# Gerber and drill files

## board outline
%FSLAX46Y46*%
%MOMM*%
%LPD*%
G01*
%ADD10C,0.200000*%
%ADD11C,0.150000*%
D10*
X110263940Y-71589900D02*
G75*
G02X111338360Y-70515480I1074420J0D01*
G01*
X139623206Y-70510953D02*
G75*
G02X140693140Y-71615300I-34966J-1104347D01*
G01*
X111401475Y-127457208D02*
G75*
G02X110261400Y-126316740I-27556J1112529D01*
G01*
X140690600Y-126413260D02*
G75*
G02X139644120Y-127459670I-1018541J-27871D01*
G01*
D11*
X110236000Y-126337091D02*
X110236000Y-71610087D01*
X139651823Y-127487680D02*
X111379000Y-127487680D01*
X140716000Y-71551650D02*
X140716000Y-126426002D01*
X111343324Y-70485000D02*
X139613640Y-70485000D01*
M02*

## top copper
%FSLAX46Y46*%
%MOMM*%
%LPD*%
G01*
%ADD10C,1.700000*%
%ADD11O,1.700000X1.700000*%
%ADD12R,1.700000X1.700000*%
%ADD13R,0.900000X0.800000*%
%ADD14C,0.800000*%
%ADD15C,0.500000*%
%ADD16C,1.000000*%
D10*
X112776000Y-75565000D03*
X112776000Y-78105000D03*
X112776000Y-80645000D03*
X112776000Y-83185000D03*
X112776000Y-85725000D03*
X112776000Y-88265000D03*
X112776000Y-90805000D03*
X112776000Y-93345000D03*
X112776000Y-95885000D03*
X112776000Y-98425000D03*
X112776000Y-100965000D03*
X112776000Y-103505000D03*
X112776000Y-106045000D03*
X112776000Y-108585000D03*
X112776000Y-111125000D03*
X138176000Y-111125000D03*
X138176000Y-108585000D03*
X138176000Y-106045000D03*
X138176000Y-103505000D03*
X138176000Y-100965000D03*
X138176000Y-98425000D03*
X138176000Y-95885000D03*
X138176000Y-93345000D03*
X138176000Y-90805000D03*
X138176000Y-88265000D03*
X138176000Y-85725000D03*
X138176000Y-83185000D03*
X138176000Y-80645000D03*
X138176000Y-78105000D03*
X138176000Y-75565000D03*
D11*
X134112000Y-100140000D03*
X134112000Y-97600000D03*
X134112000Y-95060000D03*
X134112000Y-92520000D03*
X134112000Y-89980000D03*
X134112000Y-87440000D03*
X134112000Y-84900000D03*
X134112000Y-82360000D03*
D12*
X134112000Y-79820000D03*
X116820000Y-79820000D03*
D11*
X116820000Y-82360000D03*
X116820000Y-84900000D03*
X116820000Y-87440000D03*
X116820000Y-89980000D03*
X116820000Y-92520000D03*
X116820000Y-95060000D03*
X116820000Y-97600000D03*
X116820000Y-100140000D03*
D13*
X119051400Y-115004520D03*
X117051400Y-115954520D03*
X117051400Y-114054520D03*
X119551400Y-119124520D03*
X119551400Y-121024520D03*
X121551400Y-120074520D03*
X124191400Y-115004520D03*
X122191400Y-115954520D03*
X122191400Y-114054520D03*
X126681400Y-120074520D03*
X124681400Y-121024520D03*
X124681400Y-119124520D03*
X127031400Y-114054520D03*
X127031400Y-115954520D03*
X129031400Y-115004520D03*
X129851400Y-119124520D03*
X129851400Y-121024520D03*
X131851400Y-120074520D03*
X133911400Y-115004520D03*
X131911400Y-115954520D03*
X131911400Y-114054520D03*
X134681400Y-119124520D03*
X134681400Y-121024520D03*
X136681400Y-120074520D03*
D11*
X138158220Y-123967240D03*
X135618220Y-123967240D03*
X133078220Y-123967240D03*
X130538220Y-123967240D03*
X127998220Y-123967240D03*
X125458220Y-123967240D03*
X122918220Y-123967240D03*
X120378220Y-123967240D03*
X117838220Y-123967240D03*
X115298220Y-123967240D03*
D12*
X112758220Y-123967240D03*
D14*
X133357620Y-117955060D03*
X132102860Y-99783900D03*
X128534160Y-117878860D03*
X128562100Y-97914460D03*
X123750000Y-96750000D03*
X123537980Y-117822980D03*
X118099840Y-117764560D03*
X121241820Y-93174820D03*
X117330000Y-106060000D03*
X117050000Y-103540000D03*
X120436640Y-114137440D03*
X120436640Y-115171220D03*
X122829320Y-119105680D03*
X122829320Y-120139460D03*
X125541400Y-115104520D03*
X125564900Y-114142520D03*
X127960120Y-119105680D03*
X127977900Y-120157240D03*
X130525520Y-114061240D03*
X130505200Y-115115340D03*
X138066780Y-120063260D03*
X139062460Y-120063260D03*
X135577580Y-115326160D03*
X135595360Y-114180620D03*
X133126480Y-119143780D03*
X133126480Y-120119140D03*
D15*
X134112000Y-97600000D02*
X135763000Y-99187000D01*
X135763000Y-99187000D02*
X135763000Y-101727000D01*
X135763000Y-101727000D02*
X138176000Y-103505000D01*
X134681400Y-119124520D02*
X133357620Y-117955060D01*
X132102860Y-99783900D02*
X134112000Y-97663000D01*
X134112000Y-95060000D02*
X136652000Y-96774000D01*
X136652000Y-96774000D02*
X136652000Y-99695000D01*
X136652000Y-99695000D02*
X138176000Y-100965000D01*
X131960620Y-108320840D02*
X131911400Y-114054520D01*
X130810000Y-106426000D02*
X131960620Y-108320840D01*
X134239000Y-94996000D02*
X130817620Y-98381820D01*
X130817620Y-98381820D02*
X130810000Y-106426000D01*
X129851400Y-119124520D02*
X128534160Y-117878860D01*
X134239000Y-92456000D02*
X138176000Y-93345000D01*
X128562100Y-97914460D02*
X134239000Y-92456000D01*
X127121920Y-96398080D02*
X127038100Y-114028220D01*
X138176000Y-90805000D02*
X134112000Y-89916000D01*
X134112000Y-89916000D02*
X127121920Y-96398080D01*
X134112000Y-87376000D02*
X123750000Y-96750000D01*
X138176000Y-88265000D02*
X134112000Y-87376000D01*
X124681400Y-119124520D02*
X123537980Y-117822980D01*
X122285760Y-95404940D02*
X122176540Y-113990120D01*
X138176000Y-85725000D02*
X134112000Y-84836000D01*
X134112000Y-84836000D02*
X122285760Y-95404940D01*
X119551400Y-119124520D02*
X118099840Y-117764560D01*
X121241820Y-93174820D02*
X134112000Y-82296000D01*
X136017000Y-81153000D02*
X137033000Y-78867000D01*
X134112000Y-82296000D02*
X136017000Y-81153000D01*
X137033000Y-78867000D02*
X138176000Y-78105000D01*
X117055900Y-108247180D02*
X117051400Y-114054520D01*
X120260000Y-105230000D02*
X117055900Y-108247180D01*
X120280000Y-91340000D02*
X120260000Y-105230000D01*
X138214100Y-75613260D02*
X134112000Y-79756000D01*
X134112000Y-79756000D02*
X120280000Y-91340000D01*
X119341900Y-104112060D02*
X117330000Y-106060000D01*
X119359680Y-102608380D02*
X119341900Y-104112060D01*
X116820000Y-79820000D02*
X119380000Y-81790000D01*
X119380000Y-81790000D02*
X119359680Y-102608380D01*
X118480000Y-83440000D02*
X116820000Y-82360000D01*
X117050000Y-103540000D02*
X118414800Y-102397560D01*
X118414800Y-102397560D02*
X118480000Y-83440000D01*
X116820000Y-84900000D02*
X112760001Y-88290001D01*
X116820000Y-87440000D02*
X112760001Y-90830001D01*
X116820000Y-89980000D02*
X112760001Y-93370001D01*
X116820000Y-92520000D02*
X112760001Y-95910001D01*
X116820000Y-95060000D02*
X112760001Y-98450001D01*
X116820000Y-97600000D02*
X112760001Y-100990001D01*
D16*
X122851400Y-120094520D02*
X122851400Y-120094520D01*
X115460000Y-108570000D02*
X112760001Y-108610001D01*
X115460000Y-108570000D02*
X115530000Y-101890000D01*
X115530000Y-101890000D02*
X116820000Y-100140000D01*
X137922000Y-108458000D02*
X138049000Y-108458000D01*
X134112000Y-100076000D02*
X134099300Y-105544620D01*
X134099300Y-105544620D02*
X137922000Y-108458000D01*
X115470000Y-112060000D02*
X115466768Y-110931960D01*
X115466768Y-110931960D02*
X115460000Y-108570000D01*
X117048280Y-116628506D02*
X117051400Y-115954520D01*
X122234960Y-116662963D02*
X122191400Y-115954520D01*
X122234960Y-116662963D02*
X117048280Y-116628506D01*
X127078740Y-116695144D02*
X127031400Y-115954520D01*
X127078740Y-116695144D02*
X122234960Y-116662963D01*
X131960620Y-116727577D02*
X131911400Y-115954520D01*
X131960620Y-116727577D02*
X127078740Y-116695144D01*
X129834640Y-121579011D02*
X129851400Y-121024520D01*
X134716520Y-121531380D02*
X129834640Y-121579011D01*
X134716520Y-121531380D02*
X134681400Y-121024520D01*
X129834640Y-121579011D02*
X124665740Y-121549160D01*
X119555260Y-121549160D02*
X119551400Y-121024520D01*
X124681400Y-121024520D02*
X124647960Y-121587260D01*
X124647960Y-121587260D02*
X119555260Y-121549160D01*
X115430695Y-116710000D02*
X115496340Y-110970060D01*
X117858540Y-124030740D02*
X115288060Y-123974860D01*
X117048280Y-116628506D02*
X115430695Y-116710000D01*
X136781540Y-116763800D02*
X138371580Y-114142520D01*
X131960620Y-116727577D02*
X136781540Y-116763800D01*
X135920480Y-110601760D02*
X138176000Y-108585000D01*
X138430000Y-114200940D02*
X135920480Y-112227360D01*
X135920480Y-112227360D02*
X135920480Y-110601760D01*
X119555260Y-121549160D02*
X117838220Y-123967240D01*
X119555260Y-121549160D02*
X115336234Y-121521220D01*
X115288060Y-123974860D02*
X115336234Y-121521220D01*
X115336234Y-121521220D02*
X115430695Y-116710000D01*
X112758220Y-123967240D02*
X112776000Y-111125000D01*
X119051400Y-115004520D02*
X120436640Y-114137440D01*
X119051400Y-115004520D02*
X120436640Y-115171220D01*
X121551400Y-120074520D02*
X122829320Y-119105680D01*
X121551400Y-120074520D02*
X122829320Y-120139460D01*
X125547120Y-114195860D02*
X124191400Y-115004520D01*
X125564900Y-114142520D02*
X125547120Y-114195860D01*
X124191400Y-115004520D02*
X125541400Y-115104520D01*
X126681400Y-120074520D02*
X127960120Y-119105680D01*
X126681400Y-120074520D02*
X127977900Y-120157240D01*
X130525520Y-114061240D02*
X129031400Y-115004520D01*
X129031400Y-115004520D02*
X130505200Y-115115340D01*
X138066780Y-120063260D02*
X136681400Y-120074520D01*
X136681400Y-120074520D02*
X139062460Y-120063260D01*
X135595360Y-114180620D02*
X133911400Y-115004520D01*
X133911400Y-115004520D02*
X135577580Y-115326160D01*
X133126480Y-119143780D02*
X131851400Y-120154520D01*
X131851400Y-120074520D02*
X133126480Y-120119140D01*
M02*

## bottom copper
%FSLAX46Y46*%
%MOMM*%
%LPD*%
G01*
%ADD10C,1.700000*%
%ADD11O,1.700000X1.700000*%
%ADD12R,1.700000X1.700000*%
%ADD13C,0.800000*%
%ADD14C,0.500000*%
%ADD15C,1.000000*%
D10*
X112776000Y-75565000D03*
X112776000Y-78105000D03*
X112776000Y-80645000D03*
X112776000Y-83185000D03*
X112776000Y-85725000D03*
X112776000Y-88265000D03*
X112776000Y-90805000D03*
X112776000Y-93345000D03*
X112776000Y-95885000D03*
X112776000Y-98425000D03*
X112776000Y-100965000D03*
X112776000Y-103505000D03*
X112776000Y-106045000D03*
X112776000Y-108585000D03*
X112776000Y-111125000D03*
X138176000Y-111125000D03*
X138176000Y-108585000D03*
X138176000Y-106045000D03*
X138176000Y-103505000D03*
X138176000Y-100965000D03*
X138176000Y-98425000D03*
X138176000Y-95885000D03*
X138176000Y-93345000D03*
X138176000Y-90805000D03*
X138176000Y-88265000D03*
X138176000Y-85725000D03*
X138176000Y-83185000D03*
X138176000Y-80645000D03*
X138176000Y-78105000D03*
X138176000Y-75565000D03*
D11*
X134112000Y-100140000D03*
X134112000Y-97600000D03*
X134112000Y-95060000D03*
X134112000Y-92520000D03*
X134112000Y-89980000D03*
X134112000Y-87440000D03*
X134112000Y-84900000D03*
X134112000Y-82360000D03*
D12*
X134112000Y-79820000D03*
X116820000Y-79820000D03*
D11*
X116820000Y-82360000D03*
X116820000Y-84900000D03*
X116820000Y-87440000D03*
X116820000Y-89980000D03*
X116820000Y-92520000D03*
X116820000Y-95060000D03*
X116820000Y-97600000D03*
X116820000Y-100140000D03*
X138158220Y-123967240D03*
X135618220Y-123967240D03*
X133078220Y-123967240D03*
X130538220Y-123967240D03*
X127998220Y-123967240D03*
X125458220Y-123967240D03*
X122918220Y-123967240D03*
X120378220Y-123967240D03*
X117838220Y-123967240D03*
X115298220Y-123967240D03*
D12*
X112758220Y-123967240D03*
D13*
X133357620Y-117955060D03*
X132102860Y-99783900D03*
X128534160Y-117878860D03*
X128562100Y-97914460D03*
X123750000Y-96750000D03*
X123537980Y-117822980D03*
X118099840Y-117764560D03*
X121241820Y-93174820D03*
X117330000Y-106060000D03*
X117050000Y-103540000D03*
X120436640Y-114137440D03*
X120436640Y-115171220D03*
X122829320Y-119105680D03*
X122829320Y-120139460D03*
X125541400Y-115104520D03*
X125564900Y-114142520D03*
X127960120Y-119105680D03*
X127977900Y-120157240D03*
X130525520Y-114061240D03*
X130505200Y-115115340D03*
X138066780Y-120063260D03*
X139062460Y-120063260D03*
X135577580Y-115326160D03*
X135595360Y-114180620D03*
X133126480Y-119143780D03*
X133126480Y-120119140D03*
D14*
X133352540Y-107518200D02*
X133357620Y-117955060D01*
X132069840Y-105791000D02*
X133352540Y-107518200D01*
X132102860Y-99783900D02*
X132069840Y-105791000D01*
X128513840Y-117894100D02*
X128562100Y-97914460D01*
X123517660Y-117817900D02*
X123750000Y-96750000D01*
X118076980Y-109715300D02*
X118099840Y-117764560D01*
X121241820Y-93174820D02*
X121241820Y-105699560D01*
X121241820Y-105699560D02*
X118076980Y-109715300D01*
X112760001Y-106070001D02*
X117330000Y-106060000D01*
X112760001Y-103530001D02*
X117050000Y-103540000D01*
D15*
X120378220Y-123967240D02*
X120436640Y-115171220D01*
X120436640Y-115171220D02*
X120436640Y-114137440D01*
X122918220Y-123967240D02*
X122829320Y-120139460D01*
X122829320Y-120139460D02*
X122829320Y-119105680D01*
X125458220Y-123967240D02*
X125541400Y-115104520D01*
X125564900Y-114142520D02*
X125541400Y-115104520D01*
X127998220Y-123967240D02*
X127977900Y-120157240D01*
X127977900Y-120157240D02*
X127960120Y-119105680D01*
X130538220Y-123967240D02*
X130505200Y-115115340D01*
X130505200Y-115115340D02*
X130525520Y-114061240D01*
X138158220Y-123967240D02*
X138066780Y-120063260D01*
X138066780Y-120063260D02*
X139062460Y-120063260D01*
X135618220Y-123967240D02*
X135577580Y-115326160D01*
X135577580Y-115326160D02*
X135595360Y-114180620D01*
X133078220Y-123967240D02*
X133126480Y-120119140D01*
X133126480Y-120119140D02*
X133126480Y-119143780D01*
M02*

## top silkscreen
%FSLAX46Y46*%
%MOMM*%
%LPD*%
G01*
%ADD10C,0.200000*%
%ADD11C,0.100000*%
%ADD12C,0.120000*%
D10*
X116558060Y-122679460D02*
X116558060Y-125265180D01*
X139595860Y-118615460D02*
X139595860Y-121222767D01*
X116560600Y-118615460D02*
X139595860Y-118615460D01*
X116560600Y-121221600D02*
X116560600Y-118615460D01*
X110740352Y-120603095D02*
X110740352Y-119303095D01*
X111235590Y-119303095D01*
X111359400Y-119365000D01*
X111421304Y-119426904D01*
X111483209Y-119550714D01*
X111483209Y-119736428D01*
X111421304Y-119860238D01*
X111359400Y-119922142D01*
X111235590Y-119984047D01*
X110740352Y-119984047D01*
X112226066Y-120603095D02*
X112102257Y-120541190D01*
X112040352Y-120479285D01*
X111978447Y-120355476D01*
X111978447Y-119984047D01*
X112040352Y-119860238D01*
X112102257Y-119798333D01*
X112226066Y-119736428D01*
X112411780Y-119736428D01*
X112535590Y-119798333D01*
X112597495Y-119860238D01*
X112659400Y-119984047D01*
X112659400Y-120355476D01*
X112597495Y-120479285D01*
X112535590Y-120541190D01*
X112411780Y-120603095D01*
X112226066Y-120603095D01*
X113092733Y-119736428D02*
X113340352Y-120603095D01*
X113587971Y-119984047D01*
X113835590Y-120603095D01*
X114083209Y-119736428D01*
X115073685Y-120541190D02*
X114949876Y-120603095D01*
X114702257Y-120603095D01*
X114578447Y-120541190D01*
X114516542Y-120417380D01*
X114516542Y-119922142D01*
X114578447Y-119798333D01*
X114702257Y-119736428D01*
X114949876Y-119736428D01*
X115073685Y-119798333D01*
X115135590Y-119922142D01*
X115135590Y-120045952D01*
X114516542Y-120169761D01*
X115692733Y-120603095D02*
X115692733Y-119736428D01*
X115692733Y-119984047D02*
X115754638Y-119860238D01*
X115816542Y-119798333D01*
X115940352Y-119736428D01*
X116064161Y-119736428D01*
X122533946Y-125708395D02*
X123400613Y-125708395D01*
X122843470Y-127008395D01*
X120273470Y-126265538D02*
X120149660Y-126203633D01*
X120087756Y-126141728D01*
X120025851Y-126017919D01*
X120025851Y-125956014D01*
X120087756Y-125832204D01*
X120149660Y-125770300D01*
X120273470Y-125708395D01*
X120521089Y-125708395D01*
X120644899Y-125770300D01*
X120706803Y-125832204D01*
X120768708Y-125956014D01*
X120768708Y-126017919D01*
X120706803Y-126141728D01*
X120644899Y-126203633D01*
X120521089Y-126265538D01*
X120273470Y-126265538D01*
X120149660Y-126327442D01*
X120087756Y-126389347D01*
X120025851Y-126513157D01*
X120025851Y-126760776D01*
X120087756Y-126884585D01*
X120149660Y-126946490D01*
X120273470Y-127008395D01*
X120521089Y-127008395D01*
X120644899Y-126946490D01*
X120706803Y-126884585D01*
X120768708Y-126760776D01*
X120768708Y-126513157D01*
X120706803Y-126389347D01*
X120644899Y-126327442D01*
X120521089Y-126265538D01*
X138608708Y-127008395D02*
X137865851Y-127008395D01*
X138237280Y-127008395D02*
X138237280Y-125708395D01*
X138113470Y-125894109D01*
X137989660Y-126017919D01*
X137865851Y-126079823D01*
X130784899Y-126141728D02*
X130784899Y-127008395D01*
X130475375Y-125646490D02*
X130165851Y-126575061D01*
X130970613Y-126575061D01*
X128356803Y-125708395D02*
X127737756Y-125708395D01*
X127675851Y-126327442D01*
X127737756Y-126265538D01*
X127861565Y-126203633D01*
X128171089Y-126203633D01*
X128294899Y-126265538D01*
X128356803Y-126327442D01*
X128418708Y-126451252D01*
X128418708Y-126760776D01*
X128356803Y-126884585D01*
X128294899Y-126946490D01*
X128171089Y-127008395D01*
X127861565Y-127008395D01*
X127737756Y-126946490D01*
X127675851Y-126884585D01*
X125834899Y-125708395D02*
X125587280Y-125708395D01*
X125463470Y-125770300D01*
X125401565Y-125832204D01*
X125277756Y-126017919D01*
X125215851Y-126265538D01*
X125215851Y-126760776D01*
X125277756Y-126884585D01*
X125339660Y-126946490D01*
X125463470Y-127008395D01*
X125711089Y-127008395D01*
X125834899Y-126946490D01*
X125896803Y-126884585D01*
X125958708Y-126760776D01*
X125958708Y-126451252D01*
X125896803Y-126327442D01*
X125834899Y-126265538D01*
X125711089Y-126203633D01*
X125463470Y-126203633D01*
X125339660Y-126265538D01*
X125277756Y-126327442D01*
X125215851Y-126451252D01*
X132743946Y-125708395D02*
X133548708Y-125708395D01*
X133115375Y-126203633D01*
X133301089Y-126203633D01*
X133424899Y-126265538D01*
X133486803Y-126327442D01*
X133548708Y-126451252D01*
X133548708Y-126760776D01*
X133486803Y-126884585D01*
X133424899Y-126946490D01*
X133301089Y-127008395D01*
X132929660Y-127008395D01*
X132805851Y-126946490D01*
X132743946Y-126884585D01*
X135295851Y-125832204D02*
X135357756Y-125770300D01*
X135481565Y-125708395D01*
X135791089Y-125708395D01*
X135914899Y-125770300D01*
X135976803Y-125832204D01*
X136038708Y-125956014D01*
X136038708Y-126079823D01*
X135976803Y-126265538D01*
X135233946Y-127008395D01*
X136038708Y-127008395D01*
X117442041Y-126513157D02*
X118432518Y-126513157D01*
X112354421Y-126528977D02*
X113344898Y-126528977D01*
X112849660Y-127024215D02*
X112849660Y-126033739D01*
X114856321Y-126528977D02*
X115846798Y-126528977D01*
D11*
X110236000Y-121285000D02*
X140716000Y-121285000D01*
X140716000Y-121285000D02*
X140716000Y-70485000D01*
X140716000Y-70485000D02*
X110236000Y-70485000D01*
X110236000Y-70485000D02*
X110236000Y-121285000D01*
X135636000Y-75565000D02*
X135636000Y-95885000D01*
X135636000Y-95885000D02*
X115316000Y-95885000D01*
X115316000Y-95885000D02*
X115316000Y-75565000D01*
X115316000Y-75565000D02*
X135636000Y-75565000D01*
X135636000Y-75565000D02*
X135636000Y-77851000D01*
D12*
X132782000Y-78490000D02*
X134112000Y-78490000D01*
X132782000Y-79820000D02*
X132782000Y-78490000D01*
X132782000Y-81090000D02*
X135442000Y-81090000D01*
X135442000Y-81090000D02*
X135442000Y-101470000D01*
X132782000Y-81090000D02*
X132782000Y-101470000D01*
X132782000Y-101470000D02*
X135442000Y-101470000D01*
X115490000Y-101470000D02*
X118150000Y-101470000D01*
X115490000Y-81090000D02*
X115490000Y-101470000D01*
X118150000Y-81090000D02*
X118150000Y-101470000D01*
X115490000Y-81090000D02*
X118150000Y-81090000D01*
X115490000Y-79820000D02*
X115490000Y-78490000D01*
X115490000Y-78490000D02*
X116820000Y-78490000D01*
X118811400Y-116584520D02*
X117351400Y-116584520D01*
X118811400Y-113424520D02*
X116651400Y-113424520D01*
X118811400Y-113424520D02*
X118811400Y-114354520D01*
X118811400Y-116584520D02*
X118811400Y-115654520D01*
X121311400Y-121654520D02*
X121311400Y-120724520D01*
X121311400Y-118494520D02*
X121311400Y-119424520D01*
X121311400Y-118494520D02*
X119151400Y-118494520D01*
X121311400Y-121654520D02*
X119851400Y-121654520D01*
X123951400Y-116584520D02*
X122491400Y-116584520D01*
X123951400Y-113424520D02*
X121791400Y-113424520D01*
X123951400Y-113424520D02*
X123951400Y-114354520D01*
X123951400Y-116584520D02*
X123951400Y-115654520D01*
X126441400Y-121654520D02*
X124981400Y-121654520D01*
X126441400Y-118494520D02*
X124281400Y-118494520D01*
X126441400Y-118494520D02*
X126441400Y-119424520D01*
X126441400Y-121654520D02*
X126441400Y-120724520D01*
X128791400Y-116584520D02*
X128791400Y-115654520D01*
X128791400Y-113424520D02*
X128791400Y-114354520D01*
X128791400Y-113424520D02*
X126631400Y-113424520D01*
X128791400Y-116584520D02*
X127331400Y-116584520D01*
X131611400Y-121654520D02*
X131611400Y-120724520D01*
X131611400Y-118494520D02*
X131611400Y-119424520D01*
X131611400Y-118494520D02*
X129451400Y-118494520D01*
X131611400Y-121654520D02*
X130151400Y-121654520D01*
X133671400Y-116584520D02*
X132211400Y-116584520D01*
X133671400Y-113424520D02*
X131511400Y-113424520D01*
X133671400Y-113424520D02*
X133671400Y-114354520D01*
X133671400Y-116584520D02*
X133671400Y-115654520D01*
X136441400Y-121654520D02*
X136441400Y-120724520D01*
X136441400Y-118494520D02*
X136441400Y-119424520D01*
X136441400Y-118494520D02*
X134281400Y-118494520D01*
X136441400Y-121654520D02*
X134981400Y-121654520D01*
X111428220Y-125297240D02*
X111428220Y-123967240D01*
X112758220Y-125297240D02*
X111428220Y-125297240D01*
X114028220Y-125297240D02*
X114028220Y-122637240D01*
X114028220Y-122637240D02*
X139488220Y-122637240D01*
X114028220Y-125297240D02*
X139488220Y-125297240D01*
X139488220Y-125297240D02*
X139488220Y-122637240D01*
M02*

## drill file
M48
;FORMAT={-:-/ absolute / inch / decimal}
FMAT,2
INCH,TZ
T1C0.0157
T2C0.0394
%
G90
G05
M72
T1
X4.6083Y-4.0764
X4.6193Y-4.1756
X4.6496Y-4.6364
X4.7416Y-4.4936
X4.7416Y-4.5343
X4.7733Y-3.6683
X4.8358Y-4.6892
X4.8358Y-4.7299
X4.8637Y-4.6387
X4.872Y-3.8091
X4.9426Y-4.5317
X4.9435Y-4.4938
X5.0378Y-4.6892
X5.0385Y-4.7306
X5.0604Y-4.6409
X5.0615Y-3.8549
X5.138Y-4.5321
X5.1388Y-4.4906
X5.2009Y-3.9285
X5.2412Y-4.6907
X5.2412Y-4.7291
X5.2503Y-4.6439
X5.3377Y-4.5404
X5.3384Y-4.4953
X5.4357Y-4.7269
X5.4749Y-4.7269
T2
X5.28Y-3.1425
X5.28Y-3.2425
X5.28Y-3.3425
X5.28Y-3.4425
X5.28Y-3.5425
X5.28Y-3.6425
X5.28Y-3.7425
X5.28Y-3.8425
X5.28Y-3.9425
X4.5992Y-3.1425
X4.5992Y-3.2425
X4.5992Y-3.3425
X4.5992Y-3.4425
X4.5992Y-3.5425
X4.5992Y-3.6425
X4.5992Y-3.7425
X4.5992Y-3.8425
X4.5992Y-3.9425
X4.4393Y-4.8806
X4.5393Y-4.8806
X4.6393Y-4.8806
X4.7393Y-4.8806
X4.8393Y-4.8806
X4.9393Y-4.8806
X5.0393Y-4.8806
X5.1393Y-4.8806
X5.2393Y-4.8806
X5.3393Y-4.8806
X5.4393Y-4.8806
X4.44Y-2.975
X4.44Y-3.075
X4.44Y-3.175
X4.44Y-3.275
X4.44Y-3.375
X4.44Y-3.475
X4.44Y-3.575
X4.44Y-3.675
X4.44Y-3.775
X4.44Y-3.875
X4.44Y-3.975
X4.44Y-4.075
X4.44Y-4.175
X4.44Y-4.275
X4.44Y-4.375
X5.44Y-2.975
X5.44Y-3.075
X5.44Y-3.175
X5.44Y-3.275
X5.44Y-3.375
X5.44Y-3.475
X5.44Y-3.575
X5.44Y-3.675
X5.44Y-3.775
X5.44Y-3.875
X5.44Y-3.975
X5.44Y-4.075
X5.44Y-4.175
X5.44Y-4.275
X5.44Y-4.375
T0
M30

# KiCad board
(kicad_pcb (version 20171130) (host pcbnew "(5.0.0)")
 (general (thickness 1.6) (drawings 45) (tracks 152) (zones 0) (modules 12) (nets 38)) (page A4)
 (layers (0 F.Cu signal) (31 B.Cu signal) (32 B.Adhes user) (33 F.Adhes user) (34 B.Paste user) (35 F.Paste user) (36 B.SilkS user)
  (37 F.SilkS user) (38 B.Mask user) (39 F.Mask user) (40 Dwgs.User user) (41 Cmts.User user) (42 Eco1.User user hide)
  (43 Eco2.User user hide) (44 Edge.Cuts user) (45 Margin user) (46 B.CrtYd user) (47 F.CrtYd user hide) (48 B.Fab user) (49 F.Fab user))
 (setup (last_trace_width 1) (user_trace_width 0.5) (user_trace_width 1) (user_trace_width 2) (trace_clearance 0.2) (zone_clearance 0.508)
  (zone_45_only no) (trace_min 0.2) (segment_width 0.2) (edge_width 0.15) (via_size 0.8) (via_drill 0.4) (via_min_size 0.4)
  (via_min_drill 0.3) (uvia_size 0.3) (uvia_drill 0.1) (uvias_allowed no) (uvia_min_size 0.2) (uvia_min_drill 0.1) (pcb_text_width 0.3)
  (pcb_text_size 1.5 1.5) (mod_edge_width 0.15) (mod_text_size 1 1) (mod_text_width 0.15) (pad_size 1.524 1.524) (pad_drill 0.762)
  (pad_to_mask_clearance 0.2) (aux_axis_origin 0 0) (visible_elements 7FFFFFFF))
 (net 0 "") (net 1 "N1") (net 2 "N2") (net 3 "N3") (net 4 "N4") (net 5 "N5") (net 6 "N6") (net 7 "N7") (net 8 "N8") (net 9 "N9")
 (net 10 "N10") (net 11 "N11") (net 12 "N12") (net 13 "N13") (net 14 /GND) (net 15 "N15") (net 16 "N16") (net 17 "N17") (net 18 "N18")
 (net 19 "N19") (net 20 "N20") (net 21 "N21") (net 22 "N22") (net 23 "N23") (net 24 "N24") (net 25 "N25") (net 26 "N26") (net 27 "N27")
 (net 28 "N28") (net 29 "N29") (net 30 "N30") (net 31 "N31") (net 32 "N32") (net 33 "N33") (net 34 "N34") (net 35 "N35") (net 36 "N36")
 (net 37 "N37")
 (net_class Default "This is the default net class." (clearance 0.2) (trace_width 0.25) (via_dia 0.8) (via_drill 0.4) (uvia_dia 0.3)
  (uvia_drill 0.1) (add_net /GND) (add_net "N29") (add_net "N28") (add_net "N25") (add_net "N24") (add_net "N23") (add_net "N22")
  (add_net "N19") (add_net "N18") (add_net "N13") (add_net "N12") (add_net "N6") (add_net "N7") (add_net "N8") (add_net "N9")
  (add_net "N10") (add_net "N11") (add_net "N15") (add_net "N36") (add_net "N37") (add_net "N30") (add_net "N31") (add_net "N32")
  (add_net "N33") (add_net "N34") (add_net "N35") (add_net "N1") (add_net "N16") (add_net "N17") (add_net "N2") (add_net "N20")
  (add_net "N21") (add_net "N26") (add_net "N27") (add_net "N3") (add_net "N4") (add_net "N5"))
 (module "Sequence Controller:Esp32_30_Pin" (layer F.Cu) (at 125.476 93.345)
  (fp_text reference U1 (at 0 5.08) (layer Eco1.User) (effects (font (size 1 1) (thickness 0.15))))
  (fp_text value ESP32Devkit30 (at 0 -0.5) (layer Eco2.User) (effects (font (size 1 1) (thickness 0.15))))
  (fp_line (start -15.24 27.94) (end 15.24 27.94) (layer F.SilkS) (width 0.1))
  (fp_line (start 15.24 27.94) (end 15.24 -22.86) (layer F.SilkS) (width 0.1))
  (fp_line (start 15.24 -22.86) (end -15.24 -22.86) (layer F.SilkS) (width 0.1))
  (fp_line (start -15.24 -22.86) (end -15.24 27.94) (layer F.SilkS) (width 0.1))
  (fp_line (start 10.16 -17.78) (end 10.16 2.54) (layer F.SilkS) (width 0.1))
  (fp_line (start 10.16 2.54) (end -10.16 2.54) (layer F.SilkS) (width 0.1))
  (fp_line (start -10.16 2.54) (end -10.16 -17.78) (layer F.SilkS) (width 0.1))
  (fp_line (start -10.16 -17.78) (end 10.16 -17.78) (layer F.SilkS) (width 0.1))
  (fp_line (start 10.16 -17.78) (end 10.16 -15.494) (layer F.SilkS) (width 0.1))
  (pad 1 thru_hole circle (at -12.7 -17.78) (size 1.7 1.7) (drill 1) (layers *.Cu *.Mask) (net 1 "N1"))
  (pad 2 thru_hole circle (at -12.7 -15.24) (size 1.7 1.7) (drill 1) (layers *.Cu *.Mask) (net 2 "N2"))
  (pad 3 thru_hole circle (at -12.7 -12.7) (size 1.7 1.7) (drill 1) (layers *.Cu *.Mask) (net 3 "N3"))
  (pad 4 thru_hole circle (at -12.7 -10.16) (size 1.7 1.7) (drill 1) (layers *.Cu *.Mask) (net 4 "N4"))
  (pad 5 thru_hole circle (at -12.7 -7.62) (size 1.7 1.7) (drill 1) (layers *.Cu *.Mask) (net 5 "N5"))
  (pad 6 thru_hole circle (at -12.7 -5.08) (size 1.7 1.7) (drill 1) (layers *.Cu *.Mask) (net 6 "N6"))
  (pad 7 thru_hole circle (at -12.7 -2.54) (size 1.7 1.7) (drill 1) (layers *.Cu *.Mask) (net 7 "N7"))
  (pad 8 thru_hole circle (at -12.7 0) (size 1.7 1.7) (drill 1) (layers *.Cu *.Mask) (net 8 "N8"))
  (pad 9 thru_hole circle (at -12.7 2.54) (size 1.7 1.7) (drill 1) (layers *.Cu *.Mask) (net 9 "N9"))
  (pad 10 thru_hole circle (at -12.7 5.08) (size 1.7 1.7) (drill 1) (layers *.Cu *.Mask) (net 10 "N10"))
  (pad 11 thru_hole circle (at -12.7 7.62) (size 1.7 1.7) (drill 1) (layers *.Cu *.Mask) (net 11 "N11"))
  (pad 12 thru_hole circle (at -12.7 10.16) (size 1.7 1.7) (drill 1) (layers *.Cu *.Mask) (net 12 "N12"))
  (pad 13 thru_hole circle (at -12.7 12.7) (size 1.7 1.7) (drill 1) (layers *.Cu *.Mask) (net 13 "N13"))
  (pad 14 thru_hole circle (at -12.7 15.24) (size 1.7 1.7) (drill 1) (layers *.Cu *.Mask) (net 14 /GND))
  (pad 15 thru_hole circle (at -12.7 17.78) (size 1.7 1.7) (drill 1) (layers *.Cu *.Mask) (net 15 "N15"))
  (pad 16 thru_hole circle (at 12.7 17.78) (size 1.7 1.7) (drill 1) (layers *.Cu *.Mask) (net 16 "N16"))
  (pad 17 thru_hole circle (at 12.7 15.24) (size 1.7 1.7) (drill 1) (layers *.Cu *.Mask) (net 14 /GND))
  (pad 18 thru_hole circle (at 12.7 12.7) (size 1.7 1.7) (drill 1) (layers *.Cu *.Mask) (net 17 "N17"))
  (pad 19 thru_hole circle (at 12.7 10.16) (size 1.7 1.7) (drill 1) (layers *.Cu *.Mask) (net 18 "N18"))
  (pad 20 thru_hole circle (at 12.7 7.62) (size 1.7 1.7) (drill 1) (layers *.Cu *.Mask) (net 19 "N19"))
  (pad 21 thru_hole circle (at 12.7 5.08) (size 1.7 1.7) (drill 1) (layers *.Cu *.Mask) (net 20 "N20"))
  (pad 22 thru_hole circle (at 12.7 2.54) (size 1.7 1.7) (drill 1) (layers *.Cu *.Mask) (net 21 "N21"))
  (pad 23 thru_hole circle (at 12.7 0) (size 1.7 1.7) (drill 1) (layers *.Cu *.Mask) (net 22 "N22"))
  (pad 24 thru_hole circle (at 12.7 -2.54) (size 1.7 1.7) (drill 1) (layers *.Cu *.Mask) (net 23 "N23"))
  (pad 25 thru_hole circle (at 12.7 -5.08) (size 1.7 1.7) (drill 1) (layers *.Cu *.Mask) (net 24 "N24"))
  (pad 26 thru_hole circle (at 12.7 -7.62) (size 1.7 1.7) (drill 1) (layers *.Cu *.Mask) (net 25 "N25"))
  (pad 27 thru_hole circle (at 12.7 -10.16) (size 1.7 1.7) (drill 1) (layers *.Cu *.Mask) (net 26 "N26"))
  (pad 28 thru_hole circle (at 12.7 -12.7) (size 1.7 1.7) (drill 1) (layers *.Cu *.Mask) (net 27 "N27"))
  (pad 29 thru_hole circle (at 12.7 -15.24) (size 1.7 1.7) (drill 1) (layers *.Cu *.Mask) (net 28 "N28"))
  (pad 30 thru_hole circle (at 12.7 -17.78) (size 1.7 1.7) (drill 1) (layers *.Cu *.Mask) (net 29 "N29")))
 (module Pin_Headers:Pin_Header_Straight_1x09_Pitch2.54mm (layer F.Cu) (at 134.112 79.82)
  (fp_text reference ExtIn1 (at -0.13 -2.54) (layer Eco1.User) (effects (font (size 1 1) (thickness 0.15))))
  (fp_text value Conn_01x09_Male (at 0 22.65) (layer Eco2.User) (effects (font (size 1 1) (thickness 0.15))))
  (fp_line (start -1.33 -1.33) (end 0 -1.33) (layer F.SilkS) (width 0.12))
  (fp_line (start -1.33 0) (end -1.33 -1.33) (layer F.SilkS) (width 0.12))
  (fp_line (start -1.33 1.27) (end 1.33 1.27) (layer F.SilkS) (width 0.12))
  (fp_line (start 1.33 1.27) (end 1.33 21.65) (layer F.SilkS) (width 0.12))
  (fp_line (start -1.33 1.27) (end -1.33 21.65) (layer F.SilkS) (width 0.12))
  (fp_line (start -1.33 21.65) (end 1.33 21.65) (layer F.SilkS) (width 0.12))
  (pad 9 thru_hole oval (at 0 20.32) (size 1.7 1.7) (drill 1) (layers *.Cu *.Mask) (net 14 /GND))
  (pad 8 thru_hole oval (at 0 17.78) (size 1.7 1.7) (drill 1) (layers *.Cu *.Mask) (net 18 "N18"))
  (pad 7 thru_hole oval (at 0 15.24) (size 1.7 1.7) (drill 1) (layers *.Cu *.Mask) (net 19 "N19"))
  (pad 6 thru_hole oval (at 0 12.7) (size 1.7 1.7) (drill 1) (layers *.Cu *.Mask) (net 22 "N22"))
  (pad 5 thru_hole oval (at 0 10.16) (size 1.7 1.7) (drill 1) (layers *.Cu *.Mask) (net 23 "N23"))
  (pad 4 thru_hole oval (at 0 7.62) (size 1.7 1.7) (drill 1) (layers *.Cu *.Mask) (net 24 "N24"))
  (pad 3 thru_hole oval (at 0 5.08) (size 1.7 1.7) (drill 1) (layers *.Cu *.Mask) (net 25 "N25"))
  (pad 2 thru_hole oval (at 0 2.54) (size 1.7 1.7) (drill 1) (layers *.Cu *.Mask) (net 28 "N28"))
  (pad 1 thru_hole rect (at 0 0) (size 1.7 1.7) (drill 1) (layers *.Cu *.Mask) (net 29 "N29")))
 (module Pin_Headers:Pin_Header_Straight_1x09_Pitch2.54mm (layer F.Cu) (at 116.82 79.82)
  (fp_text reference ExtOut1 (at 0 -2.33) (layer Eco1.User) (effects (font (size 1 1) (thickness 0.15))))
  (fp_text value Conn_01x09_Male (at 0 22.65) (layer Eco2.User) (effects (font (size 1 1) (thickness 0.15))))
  (fp_line (start -1.33 21.65) (end 1.33 21.65) (layer F.SilkS) (width 0.12))
  (fp_line (start -1.33 1.27) (end -1.33 21.65) (layer F.SilkS) (width 0.12))
  (fp_line (start 1.33 1.27) (end 1.33 21.65) (layer F.SilkS) (width 0.12))
  (fp_line (start -1.33 1.27) (end 1.33 1.27) (layer F.SilkS) (width 0.12))
  (fp_line (start -1.33 0) (end -1.33 -1.33) (layer F.SilkS) (width 0.12))
  (fp_line (start -1.33 -1.33) (end 0 -1.33) (layer F.SilkS) (width 0.12))
  (pad 1 thru_hole rect (at 0 0) (size 1.7 1.7) (drill 1) (layers *.Cu *.Mask) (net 13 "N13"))
  (pad 2 thru_hole oval (at 0 2.54) (size 1.7 1.7) (drill 1) (layers *.Cu *.Mask) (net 12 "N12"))
  (pad 3 thru_hole oval (at 0 5.08) (size 1.7 1.7) (drill 1) (layers *.Cu *.Mask) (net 6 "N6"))
  (pad 4 thru_hole oval (at 0 7.62) (size 1.7 1.7) (drill 1) (layers *.Cu *.Mask) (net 7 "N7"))
  (pad 5 thru_hole oval (at 0 10.16) (size 1.7 1.7) (drill 1) (layers *.Cu *.Mask) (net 8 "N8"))
  (pad 6 thru_hole oval (at 0 12.7) (size 1.7 1.7) (drill 1) (layers *.Cu *.Mask) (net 9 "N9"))
  (pad 7 thru_hole oval (at 0 15.24) (size 1.7 1.7) (drill 1) (layers *.Cu *.Mask) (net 10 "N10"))
  (pad 8 thru_hole oval (at 0 17.78) (size 1.7 1.7) (drill 1) (layers *.Cu *.Mask) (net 11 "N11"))
  (pad 9 thru_hole oval (at 0 20.32) (size 1.7 1.7) (drill 1) (layers *.Cu *.Mask) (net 14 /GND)))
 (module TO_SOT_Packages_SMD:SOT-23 (layer F.Cu) (at 118.0514 115.00452)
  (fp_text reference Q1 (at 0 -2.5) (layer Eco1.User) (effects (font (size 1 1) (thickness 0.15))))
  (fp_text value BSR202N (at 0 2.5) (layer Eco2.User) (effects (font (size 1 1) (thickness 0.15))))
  (fp_line (start 0.76 1.58) (end -0.7 1.58) (layer F.SilkS) (width 0.12))
  (fp_line (start 0.76 -1.58) (end -1.4 -1.58) (layer F.SilkS) (width 0.12))
  (fp_line (start 0.76 -1.58) (end 0.76 -0.65) (layer F.SilkS) (width 0.12))
  (fp_line (start 0.76 1.58) (end 0.76 0.65) (layer F.SilkS) (width 0.12))
  (pad 3 smd rect (at 1 0) (size 0.9 0.8) (layers F.Cu F.Paste F.Mask) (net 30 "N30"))
  (pad 2 smd rect (at -1 0.95) (size 0.9 0.8) (layers F.Cu F.Paste F.Mask) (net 14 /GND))
  (pad 1 smd rect (at -1 -0.95) (size 0.9 0.8) (layers F.Cu F.Paste F.Mask) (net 29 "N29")))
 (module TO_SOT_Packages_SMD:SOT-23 (layer F.Cu) (at 120.5514 120.07452)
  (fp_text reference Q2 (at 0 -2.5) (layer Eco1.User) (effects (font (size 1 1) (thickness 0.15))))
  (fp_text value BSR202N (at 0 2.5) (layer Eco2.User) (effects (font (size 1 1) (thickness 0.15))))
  (fp_line (start 0.76 1.58) (end 0.76 0.65) (layer F.SilkS) (width 0.12))
  (fp_line (start 0.76 -1.58) (end 0.76 -0.65) (layer F.SilkS) (width 0.12))
  (fp_line (start 0.76 -1.58) (end -1.4 -1.58) (layer F.SilkS) (width 0.12))
  (fp_line (start 0.76 1.58) (end -0.7 1.58) (layer F.SilkS) (width 0.12))
  (pad 1 smd rect (at -1 -0.95) (size 0.9 0.8) (layers F.Cu F.Paste F.Mask) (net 28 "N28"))
  (pad 2 smd rect (at -1 0.95) (size 0.9 0.8) (layers F.Cu F.Paste F.Mask) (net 14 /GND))
  (pad 3 smd rect (at 1 0) (size 0.9 0.8) (layers F.Cu F.Paste F.Mask) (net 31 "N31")))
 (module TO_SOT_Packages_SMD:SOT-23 (layer F.Cu) (at 123.1914 115.00452)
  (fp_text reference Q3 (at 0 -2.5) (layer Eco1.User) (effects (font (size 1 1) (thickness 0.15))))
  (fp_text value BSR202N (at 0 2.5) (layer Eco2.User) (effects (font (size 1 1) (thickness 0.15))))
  (fp_line (start 0.76 1.58) (end -0.7 1.58) (layer F.SilkS) (width 0.12))
  (fp_line (start 0.76 -1.58) (end -1.4 -1.58) (layer F.SilkS) (width 0.12))
  (fp_line (start 0.76 -1.58) (end 0.76 -0.65) (layer F.SilkS) (width 0.12))
  (fp_line (start 0.76 1.58) (end 0.76 0.65) (layer F.SilkS) (width 0.12))
  (pad 3 smd rect (at 1 0) (size 0.9 0.8) (layers F.Cu F.Paste F.Mask) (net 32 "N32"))
  (pad 2 smd rect (at -1 0.95) (size 0.9 0.8) (layers F.Cu F.Paste F.Mask) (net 14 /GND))
  (pad 1 smd rect (at -1 -0.95) (size 0.9 0.8) (layers F.Cu F.Paste F.Mask) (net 25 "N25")))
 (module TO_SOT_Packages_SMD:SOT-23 (layer F.Cu) (at 125.6814 120.07452)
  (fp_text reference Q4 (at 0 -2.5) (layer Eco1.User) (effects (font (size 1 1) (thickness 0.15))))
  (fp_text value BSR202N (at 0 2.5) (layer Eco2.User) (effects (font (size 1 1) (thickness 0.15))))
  (fp_line (start 0.76 1.58) (end -0.7 1.58) (layer F.SilkS) (width 0.12))
  (fp_line (start 0.76 -1.58) (end -1.4 -1.58) (layer F.SilkS) (width 0.12))
  (fp_line (start 0.76 -1.58) (end 0.76 -0.65) (layer F.SilkS) (width 0.12))
  (fp_line (start 0.76 1.58) (end 0.76 0.65) (layer F.SilkS) (width 0.12))
  (pad 3 smd rect (at 1 0) (size 0.9 0.8) (layers F.Cu F.Paste F.Mask) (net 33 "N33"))
  (pad 2 smd rect (at -1 0.95) (size 0.9 0.8) (layers F.Cu F.Paste F.Mask) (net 14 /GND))
  (pad 1 smd rect (at -1 -0.95) (size 0.9 0.8) (layers F.Cu F.Paste F.Mask) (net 24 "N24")))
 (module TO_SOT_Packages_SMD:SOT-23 (layer F.Cu) (at 128.0314 115.00452)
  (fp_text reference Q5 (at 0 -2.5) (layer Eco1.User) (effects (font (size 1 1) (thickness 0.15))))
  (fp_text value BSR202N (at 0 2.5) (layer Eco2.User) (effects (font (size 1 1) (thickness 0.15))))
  (fp_line (start 0.76 1.58) (end 0.76 0.65) (layer F.SilkS) (width 0.12))
  (fp_line (start 0.76 -1.58) (end 0.76 -0.65) (layer F.SilkS) (width 0.12))
  (fp_line (start 0.76 -1.58) (end -1.4 -1.58) (layer F.SilkS) (width 0.12))
  (fp_line (start 0.76 1.58) (end -0.7 1.58) (layer F.SilkS) (width 0.12))
  (pad 1 smd rect (at -1 -0.95) (size 0.9 0.8) (layers F.Cu F.Paste F.Mask) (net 23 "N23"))
  (pad 2 smd rect (at -1 0.95) (size 0.9 0.8) (layers F.Cu F.Paste F.Mask) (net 14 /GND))
  (pad 3 smd rect (at 1 0) (size 0.9 0.8) (layers F.Cu F.Paste F.Mask) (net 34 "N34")))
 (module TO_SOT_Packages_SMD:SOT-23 (layer F.Cu) (at 130.8514 120.07452)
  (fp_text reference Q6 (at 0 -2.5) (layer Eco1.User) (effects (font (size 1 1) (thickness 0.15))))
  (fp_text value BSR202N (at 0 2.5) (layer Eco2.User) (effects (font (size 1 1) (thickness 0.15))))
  (fp_line (start 0.76 1.58) (end 0.76 0.65) (layer F.SilkS) (width 0.12))
  (fp_line (start 0.76 -1.58) (end 0.76 -0.65) (layer F.SilkS) (width 0.12))
  (fp_line (start 0.76 -1.58) (end -1.4 -1.58) (layer F.SilkS) (width 0.12))
  (fp_line (start 0.76 1.58) (end -0.7 1.58) (layer F.SilkS) (width 0.12))
  (pad 1 smd rect (at -1 -0.95) (size 0.9 0.8) (layers F.Cu F.Paste F.Mask) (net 22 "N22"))
  (pad 2 smd rect (at -1 0.95) (size 0.9 0.8) (layers F.Cu F.Paste F.Mask) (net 14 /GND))
  (pad 3 smd rect (at 1 0) (size 0.9 0.8) (layers F.Cu F.Paste F.Mask) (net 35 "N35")))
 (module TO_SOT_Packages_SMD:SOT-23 (layer F.Cu) (at 132.9114 115.00452)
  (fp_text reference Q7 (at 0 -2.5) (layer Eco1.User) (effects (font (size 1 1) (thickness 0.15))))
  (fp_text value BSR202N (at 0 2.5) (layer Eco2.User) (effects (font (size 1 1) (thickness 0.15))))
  (fp_line (start 0.76 1.58) (end -0.7 1.58) (layer F.SilkS) (width 0.12))
  (fp_line (start 0.76 -1.58) (end -1.4 -1.58) (layer F.SilkS) (width 0.12))
  (fp_line (start 0.76 -1.58) (end 0.76 -0.65) (layer F.SilkS) (width 0.12))
  (fp_line (start 0.76 1.58) (end 0.76 0.65) (layer F.SilkS) (width 0.12))
  (pad 3 smd rect (at 1 0) (size 0.9 0.8) (layers F.Cu F.Paste F.Mask) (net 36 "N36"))
  (pad 2 smd rect (at -1 0.95) (size 0.9 0.8) (layers F.Cu F.Paste F.Mask) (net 14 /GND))
  (pad 1 smd rect (at -1 -0.95) (size 0.9 0.8) (layers F.Cu F.Paste F.Mask) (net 19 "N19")))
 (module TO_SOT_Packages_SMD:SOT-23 (layer F.Cu) (at 135.6814 120.07452)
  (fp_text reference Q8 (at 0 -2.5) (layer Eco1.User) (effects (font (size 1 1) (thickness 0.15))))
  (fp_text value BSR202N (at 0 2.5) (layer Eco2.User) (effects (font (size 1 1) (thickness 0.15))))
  (fp_line (start 0.76 1.58) (end 0.76 0.65) (layer F.SilkS) (width 0.12))
  (fp_line (start 0.76 -1.58) (end 0.76 -0.65) (layer F.SilkS) (width 0.12))
  (fp_line (start 0.76 -1.58) (end -1.4 -1.58) (layer F.SilkS) (width 0.12))
  (fp_line (start 0.76 1.58) (end -0.7 1.58) (layer F.SilkS) (width 0.12))
  (pad 1 smd rect (at -1 -0.95) (size 0.9 0.8) (layers F.Cu F.Paste F.Mask) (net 18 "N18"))
  (pad 2 smd rect (at -1 0.95) (size 0.9 0.8) (layers F.Cu F.Paste F.Mask) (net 14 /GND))
  (pad 3 smd rect (at 1 0) (size 0.9 0.8) (layers F.Cu F.Paste F.Mask) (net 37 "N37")))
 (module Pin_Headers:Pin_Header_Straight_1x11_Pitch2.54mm (layer F.Cu) (at 112.75822 123.96724 90)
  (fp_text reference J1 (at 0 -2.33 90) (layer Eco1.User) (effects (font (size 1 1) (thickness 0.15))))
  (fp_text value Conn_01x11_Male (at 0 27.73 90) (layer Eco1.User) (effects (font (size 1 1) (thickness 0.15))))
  (fp_line (start -1.33 -1.33) (end 0 -1.33) (layer F.SilkS) (width 0.12))
  (fp_line (start -1.33 0) (end -1.33 -1.33) (layer F.SilkS) (width 0.12))
  (fp_line (start -1.33 1.27) (end 1.33 1.27) (layer F.SilkS) (width 0.12))
  (fp_line (start 1.33 1.27) (end 1.33 26.73) (layer F.SilkS) (width 0.12))
  (fp_line (start -1.33 1.27) (end -1.33 26.73) (layer F.SilkS) (width 0.12))
  (fp_line (start -1.33 26.73) (end 1.33 26.73) (layer F.SilkS) (width 0.12))
  (pad 11 thru_hole oval (at 0 25.4 90) (size 1.7 1.7) (drill 1) (layers *.Cu *.Mask) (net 37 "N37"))
  (pad 10 thru_hole oval (at 0 22.86 90) (size 1.7 1.7) (drill 1) (layers *.Cu *.Mask) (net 36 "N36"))
  (pad 9 thru_hole oval (at 0 20.32 90) (size 1.7 1.7) (drill 1) (layers *.Cu *.Mask) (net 35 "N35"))
  (pad 8 thru_hole oval (at 0 17.78 90) (size 1.7 1.7) (drill 1) (layers *.Cu *.Mask) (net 34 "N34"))
  (pad 7 thru_hole oval (at 0 15.24 90) (size 1.7 1.7) (drill 1) (layers *.Cu *.Mask) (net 33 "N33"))
  (pad 6 thru_hole oval (at 0 12.7 90) (size 1.7 1.7) (drill 1) (layers *.Cu *.Mask) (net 32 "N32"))
  (pad 5 thru_hole oval (at 0 10.16 90) (size 1.7 1.7) (drill 1) (layers *.Cu *.Mask) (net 31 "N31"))
  (pad 4 thru_hole oval (at 0 7.62 90) (size 1.7 1.7) (drill 1) (layers *.Cu *.Mask) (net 30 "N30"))
  (pad 3 thru_hole oval (at 0 5.08 90) (size 1.7 1.7) (drill 1) (layers *.Cu *.Mask) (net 14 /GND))
  (pad 2 thru_hole oval (at 0 2.54 90) (size 1.7 1.7) (drill 1) (layers *.Cu *.Mask) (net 14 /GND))
  (pad 1 thru_hole rect (at 0 0 90) (size 1.7 1.7) (drill 1) (layers *.Cu *.Mask) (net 15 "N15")))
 (gr_arc (start 111.33836 71.5899) (end 111.33836 70.51548) (angle -90) (layer Edge.Cuts) (width 0.2))
 (gr_arc (start 139.58824 71.6153) (end 140.69314 71.6153) (angle -88.18649146) (layer Edge.Cuts) (width 0.2))
 (gr_arc (start 111.373919 126.344679) (end 110.2614 126.31674) (angle -92.85743314) (layer Edge.Cuts) (width 0.2))
 (gr_arc (start 139.672059 126.441131) (end 139.64412 127.45967) (angle -93.13871447) (layer Edge.Cuts) (width 0.2))
 (gr_line (start 116.55806 122.67946) (end 116.55806 125.26518) (layer F.SilkS) (width 0.2))
 (gr_line (start 139.59586 118.61546) (end 139.59586 121.222767) (layer F.SilkS) (width 0.2))
 (gr_line (start 116.5606 118.61546) (end 139.59586 118.61546) (layer F.SilkS) (width 0.2))
 (gr_line (start 116.5606 121.2216) (end 116.5606 118.61546) (layer F.SilkS) (width 0.2))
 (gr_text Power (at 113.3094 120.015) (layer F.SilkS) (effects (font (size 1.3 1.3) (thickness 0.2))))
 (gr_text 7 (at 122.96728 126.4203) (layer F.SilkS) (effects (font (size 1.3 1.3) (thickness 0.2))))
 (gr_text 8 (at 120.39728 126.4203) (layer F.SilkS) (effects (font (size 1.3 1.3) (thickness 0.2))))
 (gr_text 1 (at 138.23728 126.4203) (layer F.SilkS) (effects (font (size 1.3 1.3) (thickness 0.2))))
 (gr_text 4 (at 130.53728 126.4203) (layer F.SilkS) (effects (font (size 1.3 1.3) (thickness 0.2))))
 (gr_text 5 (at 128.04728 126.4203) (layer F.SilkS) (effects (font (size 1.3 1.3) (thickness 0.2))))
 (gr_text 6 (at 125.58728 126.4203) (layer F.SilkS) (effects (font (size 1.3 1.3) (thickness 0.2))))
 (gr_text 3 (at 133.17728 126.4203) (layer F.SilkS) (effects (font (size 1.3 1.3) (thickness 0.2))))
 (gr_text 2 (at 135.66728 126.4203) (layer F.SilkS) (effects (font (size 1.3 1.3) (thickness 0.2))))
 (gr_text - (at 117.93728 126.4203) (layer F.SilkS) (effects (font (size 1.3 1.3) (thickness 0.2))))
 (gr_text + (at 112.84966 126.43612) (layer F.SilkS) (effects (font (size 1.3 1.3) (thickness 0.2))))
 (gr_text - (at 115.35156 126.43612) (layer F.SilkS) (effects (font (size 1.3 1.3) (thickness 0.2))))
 (gr_line (start 110.236 126.337091) (end 110.236 71.610087) (layer Edge.Cuts) (width 0.15))
 (gr_line (start 139.651823 127.48768) (end 111.379 127.48768) (layer Edge.Cuts) (width 0.15))
 (gr_line (start 140.716 71.55165) (end 140.716 126.426002) (layer Edge.Cuts) (width 0.15))
 (gr_line (start 111.343324 70.485) (end 139.61364 70.485) (layer Edge.Cuts) (width 0.15))
 (segment (start 134.112 97.6) (end 135.763 99.187) (width 0.5) (layer F.Cu) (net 18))
 (segment (start 135.763 99.187) (end 135.763 101.727) (width 0.5) (layer F.Cu) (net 18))
 (segment (start 135.763 101.727) (end 138.176 103.505) (width 0.5) (layer F.Cu) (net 18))
 (segment (start 134.6814 119.12452) (end 133.35762 117.95506) (width 0.5) (layer F.Cu) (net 18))
 (via (at 133.35762 117.95506) (size 0.8) (drill 0.4) (layers F.Cu B.Cu) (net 18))
 (segment (start 133.35254 107.5182) (end 133.35762 117.95506) (width 0.5) (layer B.Cu) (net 18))
 (segment (start 132.06984 105.791) (end 133.35254 107.5182) (width 0.5) (layer B.Cu) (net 18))
 (segment (start 132.10286 99.7839) (end 132.06984 105.791) (width 0.5) (layer B.Cu) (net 18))
 (via (at 132.10286 99.7839) (size 0.8) (drill 0.4) (layers F.Cu B.Cu) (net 18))
 (segment (start 132.10286 99.7839) (end 134.112 97.663) (width 0.5) (layer F.Cu) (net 18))
 (segment (start 134.112 95.06) (end 136.652 96.774) (width 0.5) (layer F.Cu) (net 19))
 (segment (start 136.652 96.774) (end 136.652 99.695) (width 0.5) (layer F.Cu) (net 19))
 (segment (start 136.652 99.695) (end 138.176 100.965) (width 0.5) (layer F.Cu) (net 19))
 (segment (start 131.96062 108.32084) (end 131.9114 114.05452) (width 0.5) (layer F.Cu) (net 19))
 (segment (start 130.81 106.426) (end 131.96062 108.32084) (width 0.5) (layer F.Cu) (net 19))
 (segment (start 134.239 94.996) (end 130.81762 98.38182) (width 0.5) (layer F.Cu) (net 19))
 (segment (start 130.81762 98.38182) (end 130.81 106.426) (width 0.5) (layer F.Cu) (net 19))
 (via (at 128.53416 117.87886) (size 0.8) (drill 0.4) (layers F.Cu B.Cu) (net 22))
 (segment (start 129.8514 119.12452) (end 128.53416 117.87886) (width 0.5) (layer F.Cu) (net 22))
 (via (at 128.5621 97.91446) (size 0.8) (drill 0.4) (layers F.Cu B.Cu) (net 22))
 (segment (start 128.51384 117.8941) (end 128.5621 97.91446) (width 0.5) (layer B.Cu) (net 22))
 (segment (start 134.239 92.456) (end 138.176 93.345) (width 0.5) (layer F.Cu) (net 22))
 (segment (start 128.5621 97.91446) (end 134.239 92.456) (width 0.5) (layer F.Cu) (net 22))
 (segment (start 127.12192 96.39808) (end 127.0381 114.02822) (width 0.5) (layer F.Cu) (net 23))
 (segment (start 138.176 90.805) (end 134.112 89.916) (width 0.5) (layer F.Cu) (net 23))
 (segment (start 134.112 89.916) (end 127.12192 96.39808) (width 0.5) (layer F.Cu) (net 23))
 (via (at 123.75 96.75) (size 0.8) (drill 0.4) (layers F.Cu B.Cu) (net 24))
 (segment (start 134.112 87.376) (end 123.75 96.75) (width 0.5) (layer F.Cu) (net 24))
 (segment (start 138.176 88.265) (end 134.112 87.376) (width 0.5) (layer F.Cu) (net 24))
 (via (at 123.53798 117.82298) (size 0.8) (drill 0.4) (layers F.Cu B.Cu) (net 24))
 (segment (start 124.6814 119.12452) (end 123.53798 117.82298) (width 0.5) (layer F.Cu) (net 24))
 (segment (start 123.51766 117.8179) (end 123.75 96.75) (width 0.5) (layer B.Cu) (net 24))
 (segment (start 122.28576 95.40494) (end 122.17654 113.99012) (width 0.5) (layer F.Cu) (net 25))
 (segment (start 138.176 85.725) (end 134.112 84.836) (width 0.5) (layer F.Cu) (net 25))
 (segment (start 134.112 84.836) (end 122.28576 95.40494) (width 0.5) (layer F.Cu) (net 25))
 (segment (start 119.5514 119.12452) (end 118.09984 117.76456) (width 0.5) (layer F.Cu) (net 28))
 (via (at 118.09984 117.76456) (size 0.8) (drill 0.4) (layers F.Cu B.Cu) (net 28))
 (segment (start 121.24182 93.17482) (end 134.112 82.296) (width 0.5) (layer F.Cu) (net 28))
 (segment (start 136.017 81.153) (end 137.033 78.867) (width 0.5) (layer F.Cu) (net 28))
 (segment (start 134.112 82.296) (end 136.017 81.153) (width 0.5) (layer F.Cu) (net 28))
 (segment (start 137.033 78.867) (end 138.176 78.105) (width 0.5) (layer F.Cu) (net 28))
 (via (at 121.24182 93.17482) (size 0.8) (drill 0.4) (layers F.Cu B.Cu) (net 28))
 (segment (start 118.07698 109.7153) (end 118.09984 117.76456) (width 0.5) (layer B.Cu) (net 28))
 (segment (start 121.24182 93.17482) (end 121.24182 105.69956) (width 0.5) (layer B.Cu) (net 28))
 (segment (start 121.24182 105.69956) (end 118.07698 109.7153) (width 0.5) (layer B.Cu) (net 28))
 (segment (start 117.0559 108.24718) (end 117.0514 114.05452) (width 0.5) (layer F.Cu) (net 29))
 (segment (start 120.26 105.23) (end 117.0559 108.24718) (width 0.5) (layer F.Cu) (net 29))
 (segment (start 120.28 91.34) (end 120.26 105.23) (width 0.5) (layer F.Cu) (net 29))
 (segment (start 138.2141 75.61326) (end 134.112 79.756) (width 0.5) (layer F.Cu) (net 29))
 (segment (start 134.112 79.756) (end 120.28 91.34) (width 0.5) (layer F.Cu) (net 29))
 (via (at 117.33 106.06) (size 0.8) (drill 0.4) (layers F.Cu B.Cu) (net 13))
 (segment (start 112.760001 106.070001) (end 117.33 106.06) (width 0.5) (layer B.Cu) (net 13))
 (segment (start 119.3419 104.11206) (end 117.33 106.06) (width 0.5) (layer F.Cu) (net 13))
 (segment (start 119.35968 102.60838) (end 119.3419 104.11206) (width 0.5) (layer F.Cu) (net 13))
 (segment (start 116.82 79.82) (end 119.38 81.79) (width 0.5) (layer F.Cu) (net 13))
 (segment (start 119.38 81.79) (end 119.35968 102.60838) (width 0.5) (layer F.Cu) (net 13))
 (via (at 117.05 103.54) (size 0.8) (drill 0.4) (layers F.Cu B.Cu) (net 12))
 (segment (start 112.760001 103.530001) (end 117.05 103.54) (width 0.5) (layer B.Cu) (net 12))
 (segment (start 118.48 83.44) (end 116.82 82.36) (width 0.5) (layer F.Cu) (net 12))
 (segment (start 117.05 103.54) (end 118.4148 102.39756) (width 0.5) (layer F.Cu) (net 12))
 (segment (start 118.4148 102.39756) (end 118.48 83.44) (width 0.5) (layer F.Cu) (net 12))
 (segment (start 116.82 84.9) (end 112.760001 88.290001) (width 0.5) (layer F.Cu) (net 6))
 (segment (start 116.82 87.44) (end 112.760001 90.830001) (width 0.5) (layer F.Cu) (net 7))
 (segment (start 116.82 89.98) (end 112.760001 93.370001) (width 0.5) (layer F.Cu) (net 8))
 (segment (start 116.82 92.52) (end 112.760001 95.910001) (width 0.5) (layer F.Cu) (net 9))
 (segment (start 116.82 95.06) (end 112.760001 98.450001) (width 0.5) (layer F.Cu) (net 10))
 (segment (start 116.82 97.6) (end 112.760001 100.990001) (width 0.5) (layer F.Cu) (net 11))
 (segment (start 122.8514 120.09452) (end 122.8514 120.09452) (width 1) (layer F.Cu) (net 31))
 (segment (start 115.46 108.57) (end 112.760001 108.610001) (width 1) (layer F.Cu) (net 14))
 (segment (start 115.46 108.57) (end 115.53 101.89) (width 1) (layer F.Cu) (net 14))
 (segment (start 115.53 101.89) (end 116.82 100.14) (width 1) (layer F.Cu) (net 14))
 (segment (start 137.922 108.458) (end 138.049 108.458) (width 1) (layer F.Cu) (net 14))
 (segment (start 134.112 100.076) (end 134.0993 105.54462) (width 1) (layer F.Cu) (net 14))
 (segment (start 134.0993 105.54462) (end 137.922 108.458) (width 1) (layer F.Cu) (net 14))
 (segment (start 115.47 112.06) (end 115.466768 110.93196) (width 1) (layer F.Cu) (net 14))
 (segment (start 115.466768 110.93196) (end 115.46 108.57) (width 1) (layer F.Cu) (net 14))
 (segment (start 117.04828 116.628506) (end 117.0514 115.95452) (width 1) (layer F.Cu) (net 14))
 (segment (start 122.23496 116.662963) (end 122.1914 115.95452) (width 1) (layer F.Cu) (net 14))
 (segment (start 122.23496 116.662963) (end 117.04828 116.628506) (width 1) (layer F.Cu) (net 14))
 (segment (start 127.07874 116.695144) (end 127.0314 115.95452) (width 1) (layer F.Cu) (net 14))
 (segment (start 127.07874 116.695144) (end 122.23496 116.662963) (width 1) (layer F.Cu) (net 14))
 (segment (start 131.96062 116.727577) (end 131.9114 115.95452) (width 1) (layer F.Cu) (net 14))
 (segment (start 131.96062 116.727577) (end 127.07874 116.695144) (width 1) (layer F.Cu) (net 14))
 (segment (start 129.83464 121.579011) (end 129.8514 121.02452) (width 1) (layer F.Cu) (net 14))
 (segment (start 134.71652 121.53138) (end 129.83464 121.579011) (width 1) (layer F.Cu) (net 14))
 (segment (start 134.71652 121.53138) (end 134.6814 121.02452) (width 1) (layer F.Cu) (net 14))
 (segment (start 129.83464 121.579011) (end 124.66574 121.54916) (width 1) (layer F.Cu) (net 14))
 (segment (start 119.55526 121.54916) (end 119.5514 121.02452) (width 1) (layer F.Cu) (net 14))
 (segment (start 124.6814 121.02452) (end 124.64796 121.58726) (width 1) (layer F.Cu) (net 14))
 (segment (start 124.64796 121.58726) (end 119.55526 121.54916) (width 1) (layer F.Cu) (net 14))
 (segment (start 115.430695 116.71) (end 115.49634 110.97006) (width 1) (layer F.Cu) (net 14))
 (segment (start 117.85854 124.03074) (end 115.28806 123.97486) (width 1) (layer F.Cu) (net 14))
 (segment (start 117.04828 116.628506) (end 115.430695 116.71) (width 1) (layer F.Cu) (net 14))
 (segment (start 136.78154 116.7638) (end 138.37158 114.14252) (width 1) (layer F.Cu) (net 14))
 (segment (start 131.96062 116.727577) (end 136.78154 116.7638) (width 1) (layer F.Cu) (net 14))
 (segment (start 135.92048 110.60176) (end 138.176 108.585) (width 1) (layer F.Cu) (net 14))
 (segment (start 138.43 114.20094) (end 135.92048 112.22736) (width 1) (layer F.Cu) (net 14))
 (segment (start 135.92048 112.22736) (end 135.92048 110.60176) (width 1) (layer F.Cu) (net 14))
 (segment (start 119.55526 121.54916) (end 117.83822 123.96724) (width 1) (layer F.Cu) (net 14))
 (segment (start 119.55526 121.54916) (end 115.336234 121.52122) (width 1) (layer F.Cu) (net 14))
 (segment (start 115.28806 123.97486) (end 115.336234 121.52122) (width 1) (layer F.Cu) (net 14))
 (segment (start 115.336234 121.52122) (end 115.430695 116.71) (width 1) (layer F.Cu) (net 14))
 (segment (start 112.75822 123.96724) (end 112.776 111.125) (width 1) (layer F.Cu) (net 15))
 (via (at 120.43664 114.13744) (size 0.8) (drill 0.4) (layers F.Cu B.Cu) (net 30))
 (segment (start 119.0514 115.00452) (end 120.43664 114.13744) (width 1) (layer F.Cu) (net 30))
 (via (at 120.43664 115.17122) (size 0.8) (drill 0.4) (layers F.Cu B.Cu) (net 30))
 (segment (start 120.37822 123.96724) (end 120.43664 115.17122) (width 1) (layer B.Cu) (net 30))
 (segment (start 119.0514 115.00452) (end 120.43664 115.17122) (width 1) (layer F.Cu) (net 30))
 (segment (start 120.43664 115.17122) (end 120.43664 114.13744) (width 1) (layer B.Cu) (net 30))
 (via (at 122.82932 119.10568) (size 0.8) (drill 0.4) (layers F.Cu B.Cu) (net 31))
 (segment (start 121.5514 120.07452) (end 122.82932 119.10568) (width 1) (layer F.Cu) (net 31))
 (via (at 122.82932 120.13946) (size 0.8) (drill 0.4) (layers F.Cu B.Cu) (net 31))
 (segment (start 122.91822 123.96724) (end 122.82932 120.13946) (width 1) (layer B.Cu) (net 31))
 (segment (start 121.5514 120.07452) (end 122.82932 120.13946) (width 1) (layer F.Cu) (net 31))
 (segment (start 122.82932 120.13946) (end 122.82932 119.10568) (width 1) (layer B.Cu) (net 31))
 (via (at 125.5414 115.10452) (size 0.8) (drill 0.4) (layers F.Cu B.Cu) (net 32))
 (via (at 125.5649 114.14252) (size 0.8) (drill 0.4) (layers F.Cu B.Cu) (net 32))
 (segment (start 125.54712 114.19586) (end 124.1914 115.00452) (width 1) (layer F.Cu) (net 32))
 (segment (start 125.5649 114.14252) (end 125.54712 114.19586) (width 1) (layer F.Cu) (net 32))
 (segment (start 125.45822 123.96724) (end 125.5414 115.10452) (width 1) (layer B.Cu) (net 32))
 (segment (start 124.1914 115.00452) (end 125.5414 115.10452) (width 1) (layer F.Cu) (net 32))
 (segment (start 125.5649 114.14252) (end 125.5414 115.10452) (width 1) (layer B.Cu) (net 32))
 (via (at 127.96012 119.10568) (size 0.8) (drill 0.4) (layers F.Cu B.Cu) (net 33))
 (segment (start 126.6814 120.07452) (end 127.96012 119.10568) (width 1) (layer F.Cu) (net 33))
 (via (at 127.9779 120.15724) (size 0.8) (drill 0.4) (layers F.Cu B.Cu) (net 33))
 (segment (start 127.99822 123.96724) (end 127.9779 120.15724) (width 1) (layer B.Cu) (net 33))
 (segment (start 126.6814 120.07452) (end 127.9779 120.15724) (width 1) (layer F.Cu) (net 33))
 (segment (start 127.9779 120.15724) (end 127.96012 119.10568) (width 1) (layer B.Cu) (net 33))
 (via (at 130.52552 114.06124) (size 0.8) (drill 0.4) (layers F.Cu B.Cu) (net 34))
 (segment (start 130.52552 114.06124) (end 129.0314 115.00452) (width 1) (layer F.Cu) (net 34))
 (via (at 130.5052 115.11534) (size 0.8) (drill 0.4) (layers F.Cu B.Cu) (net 34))
 (segment (start 130.53822 123.96724) (end 130.5052 115.11534) (width 1) (layer B.Cu) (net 34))
 (segment (start 129.0314 115.00452) (end 130.5052 115.11534) (width 1) (layer F.Cu) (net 34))
 (segment (start 130.5052 115.11534) (end 130.52552 114.06124) (width 1) (layer B.Cu) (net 34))
 (via (at 138.06678 120.06326) (size 0.8) (drill 0.4) (layers F.Cu B.Cu) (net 37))
 (via (at 139.06246 120.06326) (size 0.8) (drill 0.4) (layers F.Cu B.Cu) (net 37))
 (segment (start 138.15822 123.96724) (end 138.06678 120.06326) (width 1) (layer B.Cu) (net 37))
 (segment (start 138.06678 120.06326) (end 136.6814 120.07452) (width 1) (layer F.Cu) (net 37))
 (segment (start 136.6814 120.07452) (end 139.06246 120.06326) (width 1) (layer F.Cu) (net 37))
 (segment (start 138.06678 120.06326) (end 139.06246 120.06326) (width 1) (layer B.Cu) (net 37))
 (via (at 135.57758 115.32616) (size 0.8) (drill 0.4) (layers F.Cu B.Cu) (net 36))
 (via (at 135.59536 114.18062) (size 0.8) (drill 0.4) (layers F.Cu B.Cu) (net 36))
 (segment (start 135.59536 114.18062) (end 133.9114 115.00452) (width 1) (layer F.Cu) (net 36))
 (segment (start 135.61822 123.96724) (end 135.57758 115.32616) (width 1) (layer B.Cu) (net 36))
 (segment (start 133.9114 115.00452) (end 135.57758 115.32616) (width 1) (layer F.Cu) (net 36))
 (segment (start 135.57758 115.32616) (end 135.59536 114.18062) (width 1) (layer B.Cu) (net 36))
 (via (at 133.12648 119.14378) (size 0.8) (drill 0.4) (layers F.Cu B.Cu) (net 35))
 (segment (start 133.12648 119.14378) (end 131.8514 120.15452) (width 1) (layer F.Cu) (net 35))
 (via (at 133.12648 120.11914) (size 0.8) (drill 0.4) (layers F.Cu B.Cu) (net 35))
 (segment (start 133.07822 123.96724) (end 133.12648 120.11914) (width 1) (layer B.Cu) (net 35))
 (segment (start 131.8514 120.07452) (end 133.12648 120.11914) (width 1) (layer F.Cu) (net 35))
 (segment (start 133.12648 120.11914) (end 133.12648 119.14378) (width 1) (layer B.Cu) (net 35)))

